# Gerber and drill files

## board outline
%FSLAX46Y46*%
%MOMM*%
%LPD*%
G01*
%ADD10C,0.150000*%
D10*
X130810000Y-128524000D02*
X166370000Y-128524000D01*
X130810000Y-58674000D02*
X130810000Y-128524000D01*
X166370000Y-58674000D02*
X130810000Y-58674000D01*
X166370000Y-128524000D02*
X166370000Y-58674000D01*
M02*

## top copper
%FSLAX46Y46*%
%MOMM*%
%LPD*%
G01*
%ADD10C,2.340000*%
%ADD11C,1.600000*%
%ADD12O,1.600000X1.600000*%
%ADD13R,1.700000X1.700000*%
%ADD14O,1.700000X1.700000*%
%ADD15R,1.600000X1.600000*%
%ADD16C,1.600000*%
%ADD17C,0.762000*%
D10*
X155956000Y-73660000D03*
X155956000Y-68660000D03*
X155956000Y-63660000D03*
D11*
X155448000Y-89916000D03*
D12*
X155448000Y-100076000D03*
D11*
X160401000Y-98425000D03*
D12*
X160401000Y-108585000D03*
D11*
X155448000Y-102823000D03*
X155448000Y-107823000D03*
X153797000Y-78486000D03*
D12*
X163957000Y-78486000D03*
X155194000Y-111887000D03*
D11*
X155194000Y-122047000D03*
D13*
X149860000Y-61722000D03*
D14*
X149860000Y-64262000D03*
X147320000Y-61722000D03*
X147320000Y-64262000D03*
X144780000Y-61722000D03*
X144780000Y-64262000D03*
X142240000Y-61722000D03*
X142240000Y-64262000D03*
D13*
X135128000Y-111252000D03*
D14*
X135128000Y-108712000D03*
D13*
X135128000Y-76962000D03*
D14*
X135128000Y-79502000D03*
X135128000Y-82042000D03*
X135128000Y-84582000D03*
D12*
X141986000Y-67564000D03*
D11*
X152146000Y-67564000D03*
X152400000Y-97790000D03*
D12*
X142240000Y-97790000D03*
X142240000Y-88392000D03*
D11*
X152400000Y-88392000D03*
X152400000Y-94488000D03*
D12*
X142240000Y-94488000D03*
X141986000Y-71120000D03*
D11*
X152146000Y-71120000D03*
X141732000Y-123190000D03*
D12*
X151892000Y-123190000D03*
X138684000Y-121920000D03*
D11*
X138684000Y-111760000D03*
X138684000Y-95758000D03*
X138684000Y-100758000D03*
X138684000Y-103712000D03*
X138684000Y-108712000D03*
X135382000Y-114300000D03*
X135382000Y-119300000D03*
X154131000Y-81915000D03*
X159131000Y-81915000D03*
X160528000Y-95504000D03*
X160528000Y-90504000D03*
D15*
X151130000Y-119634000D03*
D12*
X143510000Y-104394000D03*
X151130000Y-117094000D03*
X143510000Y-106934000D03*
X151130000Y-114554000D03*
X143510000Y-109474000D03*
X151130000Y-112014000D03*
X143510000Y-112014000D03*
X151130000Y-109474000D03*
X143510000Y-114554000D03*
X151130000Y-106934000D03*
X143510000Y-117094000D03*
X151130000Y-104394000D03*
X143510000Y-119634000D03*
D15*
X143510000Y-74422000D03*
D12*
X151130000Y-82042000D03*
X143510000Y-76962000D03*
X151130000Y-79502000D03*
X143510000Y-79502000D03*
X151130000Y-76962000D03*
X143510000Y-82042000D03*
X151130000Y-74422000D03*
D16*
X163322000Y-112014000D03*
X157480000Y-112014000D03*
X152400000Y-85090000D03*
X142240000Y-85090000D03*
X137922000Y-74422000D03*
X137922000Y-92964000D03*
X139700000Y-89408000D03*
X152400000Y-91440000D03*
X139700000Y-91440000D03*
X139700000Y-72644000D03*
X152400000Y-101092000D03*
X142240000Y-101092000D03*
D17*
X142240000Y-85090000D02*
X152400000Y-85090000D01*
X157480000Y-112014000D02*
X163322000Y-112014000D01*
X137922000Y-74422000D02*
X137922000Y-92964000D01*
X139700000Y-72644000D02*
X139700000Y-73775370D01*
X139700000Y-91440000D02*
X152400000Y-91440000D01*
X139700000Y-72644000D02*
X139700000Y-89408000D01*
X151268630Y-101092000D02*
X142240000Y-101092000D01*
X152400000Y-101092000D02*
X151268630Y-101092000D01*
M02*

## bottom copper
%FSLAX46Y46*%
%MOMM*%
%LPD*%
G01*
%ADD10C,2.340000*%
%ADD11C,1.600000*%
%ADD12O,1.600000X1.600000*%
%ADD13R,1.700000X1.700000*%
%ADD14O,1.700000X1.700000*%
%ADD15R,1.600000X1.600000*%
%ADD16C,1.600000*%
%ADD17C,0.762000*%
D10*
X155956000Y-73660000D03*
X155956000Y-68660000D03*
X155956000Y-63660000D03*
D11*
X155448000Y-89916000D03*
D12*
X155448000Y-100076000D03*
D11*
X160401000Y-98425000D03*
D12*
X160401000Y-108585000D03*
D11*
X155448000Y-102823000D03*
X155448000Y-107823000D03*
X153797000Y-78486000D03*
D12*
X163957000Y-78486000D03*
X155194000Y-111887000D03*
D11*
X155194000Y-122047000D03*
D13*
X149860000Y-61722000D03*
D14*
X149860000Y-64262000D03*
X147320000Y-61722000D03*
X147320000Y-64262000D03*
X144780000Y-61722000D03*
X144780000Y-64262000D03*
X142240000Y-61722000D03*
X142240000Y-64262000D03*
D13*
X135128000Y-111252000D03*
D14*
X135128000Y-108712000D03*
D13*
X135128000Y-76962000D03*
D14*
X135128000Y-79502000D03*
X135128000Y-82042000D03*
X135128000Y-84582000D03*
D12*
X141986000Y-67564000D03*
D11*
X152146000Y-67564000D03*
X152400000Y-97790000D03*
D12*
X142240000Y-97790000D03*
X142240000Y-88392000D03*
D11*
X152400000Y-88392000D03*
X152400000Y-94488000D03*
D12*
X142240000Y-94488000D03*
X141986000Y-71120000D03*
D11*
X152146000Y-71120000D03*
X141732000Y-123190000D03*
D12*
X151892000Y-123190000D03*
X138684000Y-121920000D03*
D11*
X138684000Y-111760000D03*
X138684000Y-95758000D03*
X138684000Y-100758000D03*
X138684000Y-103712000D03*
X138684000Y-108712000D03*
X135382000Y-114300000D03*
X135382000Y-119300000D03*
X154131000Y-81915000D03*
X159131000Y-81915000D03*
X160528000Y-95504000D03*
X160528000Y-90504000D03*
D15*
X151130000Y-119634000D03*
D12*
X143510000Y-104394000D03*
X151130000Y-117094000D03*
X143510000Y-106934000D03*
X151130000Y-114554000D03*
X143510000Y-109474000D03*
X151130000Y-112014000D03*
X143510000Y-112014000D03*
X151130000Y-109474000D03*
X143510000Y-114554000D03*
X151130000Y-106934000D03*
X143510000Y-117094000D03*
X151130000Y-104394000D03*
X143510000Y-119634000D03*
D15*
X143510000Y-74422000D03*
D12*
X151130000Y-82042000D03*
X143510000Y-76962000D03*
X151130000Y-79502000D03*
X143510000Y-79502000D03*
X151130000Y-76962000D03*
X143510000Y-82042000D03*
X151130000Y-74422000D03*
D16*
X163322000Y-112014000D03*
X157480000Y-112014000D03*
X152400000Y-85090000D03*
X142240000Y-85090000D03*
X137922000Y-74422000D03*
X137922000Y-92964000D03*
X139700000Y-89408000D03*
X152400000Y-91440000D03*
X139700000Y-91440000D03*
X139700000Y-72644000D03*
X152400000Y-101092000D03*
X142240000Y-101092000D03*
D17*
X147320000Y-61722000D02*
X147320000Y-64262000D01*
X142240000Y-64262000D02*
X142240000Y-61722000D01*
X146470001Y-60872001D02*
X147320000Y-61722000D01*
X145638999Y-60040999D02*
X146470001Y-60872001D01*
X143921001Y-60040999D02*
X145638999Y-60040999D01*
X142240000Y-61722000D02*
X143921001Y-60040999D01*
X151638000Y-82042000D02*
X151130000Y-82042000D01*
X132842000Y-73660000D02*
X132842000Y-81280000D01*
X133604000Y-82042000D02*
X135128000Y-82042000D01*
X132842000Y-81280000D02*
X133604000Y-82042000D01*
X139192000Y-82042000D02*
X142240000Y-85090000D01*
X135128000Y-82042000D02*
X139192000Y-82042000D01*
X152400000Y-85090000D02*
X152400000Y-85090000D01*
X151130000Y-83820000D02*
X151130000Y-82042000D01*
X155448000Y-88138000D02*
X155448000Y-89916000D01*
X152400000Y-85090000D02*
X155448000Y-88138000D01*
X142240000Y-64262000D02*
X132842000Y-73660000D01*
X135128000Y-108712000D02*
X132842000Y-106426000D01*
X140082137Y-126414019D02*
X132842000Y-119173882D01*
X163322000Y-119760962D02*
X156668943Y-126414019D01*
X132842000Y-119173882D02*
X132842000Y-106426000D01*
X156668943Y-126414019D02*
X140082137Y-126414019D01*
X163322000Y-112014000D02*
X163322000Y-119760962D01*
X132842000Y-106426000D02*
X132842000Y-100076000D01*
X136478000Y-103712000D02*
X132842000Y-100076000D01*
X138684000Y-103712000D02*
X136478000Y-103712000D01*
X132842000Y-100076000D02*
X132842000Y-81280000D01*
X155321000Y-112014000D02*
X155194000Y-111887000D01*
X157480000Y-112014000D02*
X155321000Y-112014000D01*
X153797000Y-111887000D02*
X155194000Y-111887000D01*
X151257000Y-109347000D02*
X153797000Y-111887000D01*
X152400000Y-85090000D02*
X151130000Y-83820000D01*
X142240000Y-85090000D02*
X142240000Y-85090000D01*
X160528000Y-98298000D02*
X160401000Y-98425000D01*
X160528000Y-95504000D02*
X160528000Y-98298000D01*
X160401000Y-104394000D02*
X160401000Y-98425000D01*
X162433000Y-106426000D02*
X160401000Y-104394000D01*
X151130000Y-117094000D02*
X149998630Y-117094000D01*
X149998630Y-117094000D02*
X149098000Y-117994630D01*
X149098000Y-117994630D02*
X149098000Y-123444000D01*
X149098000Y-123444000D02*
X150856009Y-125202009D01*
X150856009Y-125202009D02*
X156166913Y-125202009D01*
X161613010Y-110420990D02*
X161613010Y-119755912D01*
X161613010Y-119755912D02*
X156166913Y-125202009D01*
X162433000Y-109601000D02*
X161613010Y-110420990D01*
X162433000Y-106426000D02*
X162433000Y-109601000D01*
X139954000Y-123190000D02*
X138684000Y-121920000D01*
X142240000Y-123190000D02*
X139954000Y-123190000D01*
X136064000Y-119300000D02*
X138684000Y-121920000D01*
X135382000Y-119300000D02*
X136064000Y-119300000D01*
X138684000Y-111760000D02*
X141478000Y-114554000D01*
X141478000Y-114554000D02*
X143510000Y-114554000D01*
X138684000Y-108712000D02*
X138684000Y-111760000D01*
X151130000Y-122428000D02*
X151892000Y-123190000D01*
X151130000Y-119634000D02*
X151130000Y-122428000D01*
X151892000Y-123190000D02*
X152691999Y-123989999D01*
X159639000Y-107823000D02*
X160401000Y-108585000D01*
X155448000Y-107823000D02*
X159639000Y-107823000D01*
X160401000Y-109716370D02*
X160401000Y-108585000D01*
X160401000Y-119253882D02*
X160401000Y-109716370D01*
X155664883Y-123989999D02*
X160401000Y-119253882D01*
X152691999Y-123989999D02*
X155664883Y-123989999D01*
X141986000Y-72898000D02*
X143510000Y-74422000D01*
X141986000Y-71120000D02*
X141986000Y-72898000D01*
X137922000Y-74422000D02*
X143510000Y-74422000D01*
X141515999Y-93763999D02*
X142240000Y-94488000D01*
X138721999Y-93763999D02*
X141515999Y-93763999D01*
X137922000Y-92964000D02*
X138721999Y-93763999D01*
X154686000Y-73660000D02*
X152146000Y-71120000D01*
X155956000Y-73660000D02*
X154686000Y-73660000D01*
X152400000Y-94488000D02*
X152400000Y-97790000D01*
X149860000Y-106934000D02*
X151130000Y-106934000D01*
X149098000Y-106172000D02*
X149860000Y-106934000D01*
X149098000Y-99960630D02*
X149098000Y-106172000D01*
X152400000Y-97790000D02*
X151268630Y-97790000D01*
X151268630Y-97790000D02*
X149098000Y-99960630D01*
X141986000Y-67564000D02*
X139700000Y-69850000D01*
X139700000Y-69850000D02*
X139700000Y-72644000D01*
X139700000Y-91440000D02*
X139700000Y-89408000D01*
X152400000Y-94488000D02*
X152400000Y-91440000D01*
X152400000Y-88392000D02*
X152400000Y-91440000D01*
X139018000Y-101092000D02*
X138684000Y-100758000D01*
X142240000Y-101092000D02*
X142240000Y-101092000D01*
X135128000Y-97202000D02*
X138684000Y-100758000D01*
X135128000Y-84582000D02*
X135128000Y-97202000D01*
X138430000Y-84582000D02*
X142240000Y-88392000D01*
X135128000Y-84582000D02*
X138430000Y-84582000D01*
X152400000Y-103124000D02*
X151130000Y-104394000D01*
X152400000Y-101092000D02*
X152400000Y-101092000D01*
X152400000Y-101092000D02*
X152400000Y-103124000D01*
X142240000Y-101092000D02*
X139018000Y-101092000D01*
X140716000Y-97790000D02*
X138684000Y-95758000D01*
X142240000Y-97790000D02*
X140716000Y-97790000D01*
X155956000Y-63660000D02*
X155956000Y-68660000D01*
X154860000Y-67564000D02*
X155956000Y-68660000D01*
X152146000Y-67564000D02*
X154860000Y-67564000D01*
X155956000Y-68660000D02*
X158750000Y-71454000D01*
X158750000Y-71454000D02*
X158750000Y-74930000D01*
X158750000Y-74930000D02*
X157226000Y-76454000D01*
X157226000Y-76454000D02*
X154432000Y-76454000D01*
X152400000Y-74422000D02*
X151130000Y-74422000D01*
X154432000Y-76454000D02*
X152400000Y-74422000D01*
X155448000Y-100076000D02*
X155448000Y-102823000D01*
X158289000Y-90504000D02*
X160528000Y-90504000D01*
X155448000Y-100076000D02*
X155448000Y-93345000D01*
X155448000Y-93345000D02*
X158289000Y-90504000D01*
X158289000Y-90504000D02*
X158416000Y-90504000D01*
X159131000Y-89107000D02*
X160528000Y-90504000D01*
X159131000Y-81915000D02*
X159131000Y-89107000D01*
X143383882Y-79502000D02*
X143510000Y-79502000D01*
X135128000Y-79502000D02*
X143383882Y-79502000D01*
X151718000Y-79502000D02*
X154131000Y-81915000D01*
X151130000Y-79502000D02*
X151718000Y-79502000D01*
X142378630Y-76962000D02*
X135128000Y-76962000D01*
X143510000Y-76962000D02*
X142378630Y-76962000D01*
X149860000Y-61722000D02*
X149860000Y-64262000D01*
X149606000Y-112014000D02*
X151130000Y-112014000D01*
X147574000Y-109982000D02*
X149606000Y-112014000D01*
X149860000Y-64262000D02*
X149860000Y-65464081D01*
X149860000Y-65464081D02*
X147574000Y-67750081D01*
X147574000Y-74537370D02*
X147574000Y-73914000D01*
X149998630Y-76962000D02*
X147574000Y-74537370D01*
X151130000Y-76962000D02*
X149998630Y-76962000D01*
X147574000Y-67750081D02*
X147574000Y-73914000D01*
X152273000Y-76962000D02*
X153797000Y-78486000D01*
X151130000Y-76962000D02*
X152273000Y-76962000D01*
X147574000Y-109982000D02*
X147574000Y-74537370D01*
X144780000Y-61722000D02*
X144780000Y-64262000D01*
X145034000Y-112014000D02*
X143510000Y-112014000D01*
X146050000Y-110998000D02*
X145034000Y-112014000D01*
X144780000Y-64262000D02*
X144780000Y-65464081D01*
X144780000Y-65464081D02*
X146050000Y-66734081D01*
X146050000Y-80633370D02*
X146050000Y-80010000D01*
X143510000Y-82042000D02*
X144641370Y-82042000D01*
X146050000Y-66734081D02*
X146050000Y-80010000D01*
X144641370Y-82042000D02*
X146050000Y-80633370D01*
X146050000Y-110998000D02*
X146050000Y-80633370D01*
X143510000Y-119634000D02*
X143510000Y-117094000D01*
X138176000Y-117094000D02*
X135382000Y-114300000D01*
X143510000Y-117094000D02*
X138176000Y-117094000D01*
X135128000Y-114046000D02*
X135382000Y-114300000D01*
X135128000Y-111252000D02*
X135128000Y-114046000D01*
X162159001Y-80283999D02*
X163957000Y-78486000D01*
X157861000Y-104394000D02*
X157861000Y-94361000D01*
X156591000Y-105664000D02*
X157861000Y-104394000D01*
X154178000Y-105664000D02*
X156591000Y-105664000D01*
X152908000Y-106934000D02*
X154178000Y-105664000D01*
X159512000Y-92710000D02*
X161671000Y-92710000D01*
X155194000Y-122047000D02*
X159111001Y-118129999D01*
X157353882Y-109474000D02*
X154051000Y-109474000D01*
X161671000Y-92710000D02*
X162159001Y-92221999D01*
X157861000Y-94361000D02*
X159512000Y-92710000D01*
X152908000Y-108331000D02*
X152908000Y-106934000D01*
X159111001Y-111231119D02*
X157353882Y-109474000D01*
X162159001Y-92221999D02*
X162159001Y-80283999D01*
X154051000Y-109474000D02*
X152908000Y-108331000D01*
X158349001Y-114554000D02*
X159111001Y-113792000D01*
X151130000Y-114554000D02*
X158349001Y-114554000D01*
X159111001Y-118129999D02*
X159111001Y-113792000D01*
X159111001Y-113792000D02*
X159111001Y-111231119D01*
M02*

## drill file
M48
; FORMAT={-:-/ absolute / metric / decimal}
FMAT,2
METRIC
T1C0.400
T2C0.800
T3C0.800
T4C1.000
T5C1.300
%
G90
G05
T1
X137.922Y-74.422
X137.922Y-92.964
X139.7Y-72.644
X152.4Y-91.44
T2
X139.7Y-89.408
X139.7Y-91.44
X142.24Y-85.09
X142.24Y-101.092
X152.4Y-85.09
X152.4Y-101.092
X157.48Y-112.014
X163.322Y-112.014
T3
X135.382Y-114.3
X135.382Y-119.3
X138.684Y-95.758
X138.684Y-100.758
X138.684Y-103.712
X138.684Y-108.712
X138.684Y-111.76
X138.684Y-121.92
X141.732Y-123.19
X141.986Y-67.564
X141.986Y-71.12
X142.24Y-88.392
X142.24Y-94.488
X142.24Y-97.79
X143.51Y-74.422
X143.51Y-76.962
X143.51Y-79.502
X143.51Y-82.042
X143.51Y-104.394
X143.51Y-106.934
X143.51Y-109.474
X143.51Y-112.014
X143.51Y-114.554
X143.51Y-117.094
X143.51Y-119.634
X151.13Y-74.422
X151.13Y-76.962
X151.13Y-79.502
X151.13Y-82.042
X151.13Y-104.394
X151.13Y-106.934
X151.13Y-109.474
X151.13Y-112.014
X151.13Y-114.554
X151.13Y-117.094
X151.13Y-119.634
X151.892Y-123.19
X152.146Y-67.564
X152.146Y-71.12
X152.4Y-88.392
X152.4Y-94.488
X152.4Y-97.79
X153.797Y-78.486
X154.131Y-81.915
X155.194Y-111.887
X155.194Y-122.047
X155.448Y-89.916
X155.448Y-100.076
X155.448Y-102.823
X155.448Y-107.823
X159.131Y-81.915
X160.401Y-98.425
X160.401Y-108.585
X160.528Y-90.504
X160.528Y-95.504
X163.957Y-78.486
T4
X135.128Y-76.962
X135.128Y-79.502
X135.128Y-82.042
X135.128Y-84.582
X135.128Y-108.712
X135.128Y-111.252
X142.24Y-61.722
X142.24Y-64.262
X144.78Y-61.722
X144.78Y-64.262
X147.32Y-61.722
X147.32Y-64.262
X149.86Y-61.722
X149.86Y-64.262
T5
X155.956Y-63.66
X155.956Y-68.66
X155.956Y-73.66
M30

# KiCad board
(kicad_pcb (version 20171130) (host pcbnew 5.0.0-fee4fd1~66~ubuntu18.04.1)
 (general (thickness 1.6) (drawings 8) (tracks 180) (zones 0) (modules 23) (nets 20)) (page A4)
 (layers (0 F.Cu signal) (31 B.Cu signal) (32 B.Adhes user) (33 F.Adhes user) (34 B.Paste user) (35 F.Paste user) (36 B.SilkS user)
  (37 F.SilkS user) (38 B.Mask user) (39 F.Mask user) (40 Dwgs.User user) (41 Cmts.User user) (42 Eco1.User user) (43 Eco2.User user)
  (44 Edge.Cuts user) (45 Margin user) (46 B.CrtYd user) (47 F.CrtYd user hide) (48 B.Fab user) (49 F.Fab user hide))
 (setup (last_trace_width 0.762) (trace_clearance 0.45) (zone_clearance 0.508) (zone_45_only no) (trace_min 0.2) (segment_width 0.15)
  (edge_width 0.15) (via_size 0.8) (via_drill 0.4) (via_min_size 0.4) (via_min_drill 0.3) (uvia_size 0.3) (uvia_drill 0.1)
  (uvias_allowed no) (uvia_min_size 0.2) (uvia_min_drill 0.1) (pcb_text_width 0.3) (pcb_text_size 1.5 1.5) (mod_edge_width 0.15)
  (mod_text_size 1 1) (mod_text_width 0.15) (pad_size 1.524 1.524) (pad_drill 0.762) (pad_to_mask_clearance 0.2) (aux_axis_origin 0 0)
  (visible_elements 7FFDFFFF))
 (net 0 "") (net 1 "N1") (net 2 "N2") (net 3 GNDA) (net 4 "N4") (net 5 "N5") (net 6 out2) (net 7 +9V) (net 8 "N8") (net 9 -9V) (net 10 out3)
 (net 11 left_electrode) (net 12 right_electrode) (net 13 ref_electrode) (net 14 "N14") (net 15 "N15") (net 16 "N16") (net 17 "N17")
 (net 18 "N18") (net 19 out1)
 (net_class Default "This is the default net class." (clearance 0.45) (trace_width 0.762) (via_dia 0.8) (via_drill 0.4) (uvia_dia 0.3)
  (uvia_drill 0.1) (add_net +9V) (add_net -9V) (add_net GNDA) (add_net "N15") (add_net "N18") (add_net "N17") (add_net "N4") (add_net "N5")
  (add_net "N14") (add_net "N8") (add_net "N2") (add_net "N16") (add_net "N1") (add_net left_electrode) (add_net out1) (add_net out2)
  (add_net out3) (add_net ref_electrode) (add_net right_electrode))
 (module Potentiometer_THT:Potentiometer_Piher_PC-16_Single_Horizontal (layer F.Cu) (at 155.956 73.66)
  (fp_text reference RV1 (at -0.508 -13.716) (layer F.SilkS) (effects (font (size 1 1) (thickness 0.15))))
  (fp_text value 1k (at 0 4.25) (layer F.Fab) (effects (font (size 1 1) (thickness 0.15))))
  (pad 1 thru_hole circle (at 0 0) (size 2.34 2.34) (drill 1.3) (layers *.Cu *.Mask) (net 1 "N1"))
  (pad 2 thru_hole circle (at 0 -5) (size 2.34 2.34) (drill 1.3) (layers *.Cu *.Mask) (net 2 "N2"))
  (pad 3 thru_hole circle (at 0 -10) (size 2.34 2.34) (drill 1.3) (layers *.Cu *.Mask) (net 2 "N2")))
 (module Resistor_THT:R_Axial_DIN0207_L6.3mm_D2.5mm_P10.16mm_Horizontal (layer F.Cu) (at 155.448 89.916 270)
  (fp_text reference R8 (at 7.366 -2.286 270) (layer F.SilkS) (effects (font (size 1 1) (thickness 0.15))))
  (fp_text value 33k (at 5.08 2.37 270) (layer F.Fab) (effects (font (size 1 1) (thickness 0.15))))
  (pad 1 thru_hole circle (at 0 0 270) (size 1.6 1.6) (drill 0.8) (layers *.Cu *.Mask) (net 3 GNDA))
  (pad 2 thru_hole oval (at 10.16 0 270) (size 1.6 1.6) (drill 0.8) (layers *.Cu *.Mask) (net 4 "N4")))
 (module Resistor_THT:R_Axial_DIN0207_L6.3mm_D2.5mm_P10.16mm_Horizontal (layer F.Cu) (at 160.401 98.425 270)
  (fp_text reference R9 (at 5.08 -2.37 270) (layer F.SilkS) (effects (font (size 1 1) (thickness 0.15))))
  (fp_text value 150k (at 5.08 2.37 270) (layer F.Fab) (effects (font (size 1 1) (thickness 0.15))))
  (pad 1 thru_hole circle (at 0 0 270) (size 1.6 1.6) (drill 0.8) (layers *.Cu *.Mask) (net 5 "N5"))
  (pad 2 thru_hole oval (at 10.16 0 270) (size 1.6 1.6) (drill 0.8) (layers *.Cu *.Mask) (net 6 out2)))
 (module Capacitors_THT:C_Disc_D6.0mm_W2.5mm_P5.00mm (layer F.Cu) (at 155.448 107.823 90)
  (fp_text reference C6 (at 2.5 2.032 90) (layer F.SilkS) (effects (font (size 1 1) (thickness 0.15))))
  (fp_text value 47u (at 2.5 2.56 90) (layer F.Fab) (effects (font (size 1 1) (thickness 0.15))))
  (pad 2 thru_hole circle (at 5 0 90) (size 1.6 1.6) (drill 0.8) (layers *.Cu *.Mask) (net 4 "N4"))
  (pad 1 thru_hole circle (at 0 0 90) (size 1.6 1.6) (drill 0.8) (layers *.Cu *.Mask) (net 6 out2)))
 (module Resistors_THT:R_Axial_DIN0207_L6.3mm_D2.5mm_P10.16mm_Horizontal (layer F.Cu) (at 153.797 78.486)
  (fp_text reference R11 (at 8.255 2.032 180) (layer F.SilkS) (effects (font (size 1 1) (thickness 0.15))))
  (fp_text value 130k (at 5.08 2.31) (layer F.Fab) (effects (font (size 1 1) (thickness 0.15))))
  (pad 1 thru_hole circle (at 0 0) (size 1.6 1.6) (drill 0.8) (layers *.Cu *.Mask) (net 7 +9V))
  (pad 2 thru_hole oval (at 10.16 0) (size 1.6 1.6) (drill 0.8) (layers *.Cu *.Mask) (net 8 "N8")))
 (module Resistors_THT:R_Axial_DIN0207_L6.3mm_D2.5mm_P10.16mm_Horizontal (layer F.Cu) (at 155.194 122.047 90)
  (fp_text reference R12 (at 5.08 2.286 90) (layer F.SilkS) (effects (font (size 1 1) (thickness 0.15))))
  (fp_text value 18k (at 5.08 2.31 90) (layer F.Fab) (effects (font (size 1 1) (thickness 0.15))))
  (pad 2 thru_hole oval (at 10.16 0 90) (size 1.6 1.6) (drill 0.8) (layers *.Cu *.Mask) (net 3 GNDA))
  (pad 1 thru_hole circle (at 0 0 90) (size 1.6 1.6) (drill 0.8) (layers *.Cu *.Mask) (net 8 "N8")))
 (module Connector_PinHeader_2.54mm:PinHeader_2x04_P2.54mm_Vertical (layer F.Cu) (at 149.86 61.722 270)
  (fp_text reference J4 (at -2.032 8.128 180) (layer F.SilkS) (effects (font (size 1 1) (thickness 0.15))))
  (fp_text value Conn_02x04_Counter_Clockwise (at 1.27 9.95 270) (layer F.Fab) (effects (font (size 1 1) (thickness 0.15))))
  (pad 1 thru_hole rect (at 0 0 270) (size 1.7 1.7) (drill 1) (layers *.Cu *.Mask) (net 7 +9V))
  (pad 2 thru_hole oval (at 2.54 0 270) (size 1.7 1.7) (drill 1) (layers *.Cu *.Mask) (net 7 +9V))
  (pad 3 thru_hole oval (at 0 2.54 270) (size 1.7 1.7) (drill 1) (layers *.Cu *.Mask) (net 3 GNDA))
  (pad 4 thru_hole oval (at 2.54 2.54 270) (size 1.7 1.7) (drill 1) (layers *.Cu *.Mask) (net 3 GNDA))
  (pad 5 thru_hole oval (at 0 5.08 270) (size 1.7 1.7) (drill 1) (layers *.Cu *.Mask) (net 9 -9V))
  (pad 6 thru_hole oval (at 2.54 5.08 270) (size 1.7 1.7) (drill 1) (layers *.Cu *.Mask) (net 9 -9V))
  (pad 7 thru_hole oval (at 0 7.62 270) (size 1.7 1.7) (drill 1) (layers *.Cu *.Mask) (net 3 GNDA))
  (pad 8 thru_hole oval (at 2.54 7.62 270) (size 1.7 1.7) (drill 1) (layers *.Cu *.Mask) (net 3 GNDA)))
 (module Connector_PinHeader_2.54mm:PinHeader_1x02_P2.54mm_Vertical (layer F.Cu) (at 135.128 111.252 180)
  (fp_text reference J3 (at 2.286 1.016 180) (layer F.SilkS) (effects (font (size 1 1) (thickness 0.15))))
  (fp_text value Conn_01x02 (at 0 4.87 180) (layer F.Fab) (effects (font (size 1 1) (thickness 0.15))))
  (pad 1 thru_hole rect (at 0 0 180) (size 1.7 1.7) (drill 1) (layers *.Cu *.Mask) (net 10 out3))
  (pad 2 thru_hole oval (at 0 2.54 180) (size 1.7 1.7) (drill 1) (layers *.Cu *.Mask) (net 3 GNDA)))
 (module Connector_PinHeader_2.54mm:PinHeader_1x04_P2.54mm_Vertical (layer F.Cu) (at 135.128 76.962)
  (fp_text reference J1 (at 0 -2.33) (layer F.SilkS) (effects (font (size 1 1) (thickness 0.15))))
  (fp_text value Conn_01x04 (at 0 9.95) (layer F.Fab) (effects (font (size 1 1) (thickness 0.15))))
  (pad 1 thru_hole rect (at 0 0) (size 1.7 1.7) (drill 1) (layers *.Cu *.Mask) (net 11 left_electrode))
  (pad 2 thru_hole oval (at 0 2.54) (size 1.7 1.7) (drill 1) (layers *.Cu *.Mask) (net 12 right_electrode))
  (pad 3 thru_hole oval (at 0 5.08) (size 1.7 1.7) (drill 1) (layers *.Cu *.Mask) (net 3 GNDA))
  (pad 4 thru_hole oval (at 0 7.62) (size 1.7 1.7) (drill 1) (layers *.Cu *.Mask) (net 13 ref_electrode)))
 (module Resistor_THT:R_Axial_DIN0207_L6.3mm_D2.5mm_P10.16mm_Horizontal (layer F.Cu) (at 152.146 67.564 180)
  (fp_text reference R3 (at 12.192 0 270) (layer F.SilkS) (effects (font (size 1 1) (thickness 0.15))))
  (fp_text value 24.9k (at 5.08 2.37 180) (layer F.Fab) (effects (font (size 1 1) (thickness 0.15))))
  (pad 2 thru_hole oval (at 10.16 0 180) (size 1.6 1.6) (drill 0.8) (layers *.Cu *.Mask) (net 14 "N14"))
  (pad 1 thru_hole circle (at 0 0 180) (size 1.6 1.6) (drill 0.8) (layers *.Cu *.Mask) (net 2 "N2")))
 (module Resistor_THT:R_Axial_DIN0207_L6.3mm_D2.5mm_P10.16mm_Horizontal (layer F.Cu) (at 152.4 97.79 180)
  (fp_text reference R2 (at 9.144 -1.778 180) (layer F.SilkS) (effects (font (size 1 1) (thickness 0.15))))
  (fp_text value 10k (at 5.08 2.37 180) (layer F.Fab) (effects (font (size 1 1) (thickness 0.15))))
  (pad 1 thru_hole circle (at 0 0 180) (size 1.6 1.6) (drill 0.8) (layers *.Cu *.Mask) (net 14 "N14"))
  (pad 2 thru_hole oval (at 10.16 0 180) (size 1.6 1.6) (drill 0.8) (layers *.Cu *.Mask) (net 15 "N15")))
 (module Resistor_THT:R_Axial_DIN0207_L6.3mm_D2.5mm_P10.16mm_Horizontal (layer F.Cu) (at 152.4 88.392 180)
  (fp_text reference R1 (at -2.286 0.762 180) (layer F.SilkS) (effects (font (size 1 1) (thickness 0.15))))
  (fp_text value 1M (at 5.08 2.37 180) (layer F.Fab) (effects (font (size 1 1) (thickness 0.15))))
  (pad 2 thru_hole oval (at 10.16 0 180) (size 1.6 1.6) (drill 0.8) (layers *.Cu *.Mask) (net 13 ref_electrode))
  (pad 1 thru_hole circle (at 0 0 180) (size 1.6 1.6) (drill 0.8) (layers *.Cu *.Mask) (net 14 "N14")))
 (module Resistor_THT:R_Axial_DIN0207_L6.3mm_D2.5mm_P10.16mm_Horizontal (layer F.Cu) (at 152.4 94.488 180)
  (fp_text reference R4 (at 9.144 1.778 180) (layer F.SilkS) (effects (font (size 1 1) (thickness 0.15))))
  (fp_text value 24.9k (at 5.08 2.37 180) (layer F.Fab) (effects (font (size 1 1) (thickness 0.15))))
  (pad 1 thru_hole circle (at 0 0 180) (size 1.6 1.6) (drill 0.8) (layers *.Cu *.Mask) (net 14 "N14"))
  (pad 2 thru_hole oval (at 10.16 0 180) (size 1.6 1.6) (drill 0.8) (layers *.Cu *.Mask) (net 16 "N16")))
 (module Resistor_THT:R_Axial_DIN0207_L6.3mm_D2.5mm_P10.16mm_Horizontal (layer F.Cu) (at 152.146 71.12 180)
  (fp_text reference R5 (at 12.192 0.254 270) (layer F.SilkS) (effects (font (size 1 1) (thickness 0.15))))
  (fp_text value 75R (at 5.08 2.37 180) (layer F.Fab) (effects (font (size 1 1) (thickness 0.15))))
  (pad 2 thru_hole oval (at 10.16 0 180) (size 1.6 1.6) (drill 0.8) (layers *.Cu *.Mask) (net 16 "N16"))
  (pad 1 thru_hole circle (at 0 0 180) (size 1.6 1.6) (drill 0.8) (layers *.Cu *.Mask) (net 1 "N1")))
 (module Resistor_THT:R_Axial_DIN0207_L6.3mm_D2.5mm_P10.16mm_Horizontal (layer F.Cu) (at 141.732 123.19)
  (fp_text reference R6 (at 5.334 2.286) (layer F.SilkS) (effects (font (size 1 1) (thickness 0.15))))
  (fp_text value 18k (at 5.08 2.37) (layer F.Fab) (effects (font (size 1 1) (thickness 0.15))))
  (pad 1 thru_hole circle (at 0 0) (size 1.6 1.6) (drill 0.8) (layers *.Cu *.Mask) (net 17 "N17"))
  (pad 2 thru_hole oval (at 10.16 0) (size 1.6 1.6) (drill 0.8) (layers *.Cu *.Mask) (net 6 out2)))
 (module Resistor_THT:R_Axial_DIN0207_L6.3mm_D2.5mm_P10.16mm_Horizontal (layer F.Cu) (at 138.684 111.76 270)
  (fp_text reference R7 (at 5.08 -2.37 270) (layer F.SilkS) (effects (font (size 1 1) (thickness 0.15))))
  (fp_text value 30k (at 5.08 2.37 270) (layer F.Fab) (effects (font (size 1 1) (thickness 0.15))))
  (pad 2 thru_hole oval (at 10.16 0 270) (size 1.6 1.6) (drill 0.8) (layers *.Cu *.Mask) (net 17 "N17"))
  (pad 1 thru_hole circle (at 0 0 270) (size 1.6 1.6) (drill 0.8) (layers *.Cu *.Mask) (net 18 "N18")))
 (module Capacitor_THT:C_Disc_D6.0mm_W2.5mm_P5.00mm (layer F.Cu) (at 138.684 95.758 270)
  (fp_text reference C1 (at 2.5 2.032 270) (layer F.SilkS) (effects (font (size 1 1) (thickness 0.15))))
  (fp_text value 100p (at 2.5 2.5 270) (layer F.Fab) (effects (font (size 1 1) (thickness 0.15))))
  (pad 1 thru_hole circle (at 0 0 270) (size 1.6 1.6) (drill 0.8) (layers *.Cu *.Mask) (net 15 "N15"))
  (pad 2 thru_hole circle (at 5 0 270) (size 1.6 1.6) (drill 0.8) (layers *.Cu *.Mask) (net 13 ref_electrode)))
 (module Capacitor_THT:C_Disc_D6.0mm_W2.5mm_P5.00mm (layer F.Cu) (at 138.684 108.712 90)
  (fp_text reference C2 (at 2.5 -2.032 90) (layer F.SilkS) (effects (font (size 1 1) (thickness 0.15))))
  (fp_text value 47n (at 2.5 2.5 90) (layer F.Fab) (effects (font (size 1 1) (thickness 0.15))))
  (pad 2 thru_hole circle (at 5 0 90) (size 1.6 1.6) (drill 0.8) (layers *.Cu *.Mask) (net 3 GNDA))
  (pad 1 thru_hole circle (at 0 0 90) (size 1.6 1.6) (drill 0.8) (layers *.Cu *.Mask) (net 18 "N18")))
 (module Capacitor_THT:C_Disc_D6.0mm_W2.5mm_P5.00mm (layer F.Cu) (at 135.382 114.3 270)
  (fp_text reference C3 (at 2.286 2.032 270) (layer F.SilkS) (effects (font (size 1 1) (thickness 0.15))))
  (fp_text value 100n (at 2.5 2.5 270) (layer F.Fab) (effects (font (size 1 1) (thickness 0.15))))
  (pad 1 thru_hole circle (at 0 0 270) (size 1.6 1.6) (drill 0.8) (layers *.Cu *.Mask) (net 10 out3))
  (pad 2 thru_hole circle (at 5 0 270) (size 1.6 1.6) (drill 0.8) (layers *.Cu *.Mask) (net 17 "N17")))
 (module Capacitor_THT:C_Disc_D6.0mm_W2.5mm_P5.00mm (layer F.Cu) (at 159.131 81.915 180)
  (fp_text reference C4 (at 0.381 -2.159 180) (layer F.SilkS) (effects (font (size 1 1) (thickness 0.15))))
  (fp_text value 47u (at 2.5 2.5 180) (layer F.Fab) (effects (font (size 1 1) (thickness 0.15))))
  (pad 2 thru_hole circle (at 5 0 180) (size 1.6 1.6) (drill 0.8) (layers *.Cu *.Mask) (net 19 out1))
  (pad 1 thru_hole circle (at 0 0 180) (size 1.6 1.6) (drill 0.8) (layers *.Cu *.Mask) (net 4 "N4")))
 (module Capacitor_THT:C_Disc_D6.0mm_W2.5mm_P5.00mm (layer F.Cu) (at 160.528 95.504 90)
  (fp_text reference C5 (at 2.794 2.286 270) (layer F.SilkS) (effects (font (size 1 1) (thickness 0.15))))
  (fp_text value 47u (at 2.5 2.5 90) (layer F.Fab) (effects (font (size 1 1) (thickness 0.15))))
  (pad 1 thru_hole circle (at 0 0 90) (size 1.6 1.6) (drill 0.8) (layers *.Cu *.Mask) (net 5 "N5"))
  (pad 2 thru_hole circle (at 5 0 90) (size 1.6 1.6) (drill 0.8) (layers *.Cu *.Mask) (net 4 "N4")))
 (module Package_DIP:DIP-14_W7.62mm (layer F.Cu) (at 151.13 119.634 180)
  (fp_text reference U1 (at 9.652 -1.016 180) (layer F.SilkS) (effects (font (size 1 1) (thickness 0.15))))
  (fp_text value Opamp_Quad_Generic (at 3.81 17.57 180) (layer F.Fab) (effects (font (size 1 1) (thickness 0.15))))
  (pad 1 thru_hole rect (at 0 0 180) (size 1.6 1.6) (drill 0.8) (layers *.Cu *.Mask) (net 6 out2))
  (pad 8 thru_hole oval (at 7.62 15.24 180) (size 1.6 1.6) (drill 0.8) (layers *.Cu *.Mask))
  (pad 2 thru_hole oval (at 0 2.54 180) (size 1.6 1.6) (drill 0.8) (layers *.Cu *.Mask) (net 5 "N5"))
  (pad 9 thru_hole oval (at 7.62 12.7 180) (size 1.6 1.6) (drill 0.8) (layers *.Cu *.Mask))
  (pad 3 thru_hole oval (at 0 5.08 180) (size 1.6 1.6) (drill 0.8) (layers *.Cu *.Mask) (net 8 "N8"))
  (pad 10 thru_hole oval (at 7.62 10.16 180) (size 1.6 1.6) (drill 0.8) (layers *.Cu *.Mask))
  (pad 4 thru_hole oval (at 0 7.62 180) (size 1.6 1.6) (drill 0.8) (layers *.Cu *.Mask) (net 7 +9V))
  (pad 11 thru_hole oval (at 7.62 7.62 180) (size 1.6 1.6) (drill 0.8) (layers *.Cu *.Mask) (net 9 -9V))
  (pad 5 thru_hole oval (at 0 10.16 180) (size 1.6 1.6) (drill 0.8) (layers *.Cu *.Mask) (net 3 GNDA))
  (pad 12 thru_hole oval (at 7.62 5.08 180) (size 1.6 1.6) (drill 0.8) (layers *.Cu *.Mask) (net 18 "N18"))
  (pad 6 thru_hole oval (at 0 12.7 180) (size 1.6 1.6) (drill 0.8) (layers *.Cu *.Mask) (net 14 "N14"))
  (pad 13 thru_hole oval (at 7.62 2.54 180) (size 1.6 1.6) (drill 0.8) (layers *.Cu *.Mask) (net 10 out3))
  (pad 7 thru_hole oval (at 0 15.24 180) (size 1.6 1.6) (drill 0.8) (layers *.Cu *.Mask) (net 13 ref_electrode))
  (pad 14 thru_hole oval (at 7.62 0 180) (size 1.6 1.6) (drill 0.8) (layers *.Cu *.Mask) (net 10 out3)))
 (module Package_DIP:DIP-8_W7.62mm (layer F.Cu) (at 143.51 74.422)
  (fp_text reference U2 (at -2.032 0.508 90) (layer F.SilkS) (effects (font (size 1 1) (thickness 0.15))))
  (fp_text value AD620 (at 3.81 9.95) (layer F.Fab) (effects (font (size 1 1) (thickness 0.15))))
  (pad 1 thru_hole rect (at 0 0) (size 1.6 1.6) (drill 0.8) (layers *.Cu *.Mask) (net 16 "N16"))
  (pad 5 thru_hole oval (at 7.62 7.62) (size 1.6 1.6) (drill 0.8) (layers *.Cu *.Mask) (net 3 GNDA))
  (pad 2 thru_hole oval (at 0 2.54) (size 1.6 1.6) (drill 0.8) (layers *.Cu *.Mask) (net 11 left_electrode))
  (pad 6 thru_hole oval (at 7.62 5.08) (size 1.6 1.6) (drill 0.8) (layers *.Cu *.Mask) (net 19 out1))
  (pad 3 thru_hole oval (at 0 5.08) (size 1.6 1.6) (drill 0.8) (layers *.Cu *.Mask) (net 12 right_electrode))
  (pad 7 thru_hole oval (at 7.62 2.54) (size 1.6 1.6) (drill 0.8) (layers *.Cu *.Mask) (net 7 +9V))
  (pad 4 thru_hole oval (at 0 7.62) (size 1.6 1.6) (drill 0.8) (layers *.Cu *.Mask) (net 9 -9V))
  (pad 8 thru_hole oval (at 7.62 0) (size 1.6 1.6) (drill 0.8) (layers *.Cu *.Mask) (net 2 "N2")))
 (gr_line (start 130.81 128.524) (end 166.37 128.524) (layer Edge.Cuts) (width 0.15))
 (gr_line (start 130.81 58.674) (end 130.81 128.524) (layer Edge.Cuts) (width 0.15))
 (gr_line (start 166.37 58.674) (end 130.81 58.674) (layer Edge.Cuts) (width 0.15))
 (gr_line (start 166.37 128.524) (end 166.37 58.674) (layer Edge.Cuts) (width 0.15))
 (via (at 163.322 112.014) (size 1.6) (drill 0.8) (layers F.Cu B.Cu) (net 3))
 (via (at 157.48 112.014) (size 1.6) (drill 0.8) (layers F.Cu B.Cu) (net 3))
 (segment (start 147.32 61.722) (end 147.32 64.262) (width 0.762) (layer B.Cu) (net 3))
 (segment (start 142.24 64.262) (end 142.24 61.722) (width 0.762) (layer B.Cu) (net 3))
 (segment (start 146.470001 60.872001) (end 147.32 61.722) (width 0.762) (layer B.Cu) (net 3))
 (segment (start 145.638999 60.040999) (end 146.470001 60.872001) (width 0.762) (layer B.Cu) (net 3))
 (segment (start 143.921001 60.040999) (end 145.638999 60.040999) (width 0.762) (layer B.Cu) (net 3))
 (segment (start 142.24 61.722) (end 143.921001 60.040999) (width 0.762) (layer B.Cu) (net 3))
 (segment (start 151.638 82.042) (end 151.13 82.042) (width 0.762) (layer B.Cu) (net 3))
 (segment (start 132.842 73.66) (end 132.842 81.28) (width 0.762) (layer B.Cu) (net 3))
 (segment (start 133.604 82.042) (end 135.128 82.042) (width 0.762) (layer B.Cu) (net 3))
 (segment (start 132.842 81.28) (end 133.604 82.042) (width 0.762) (layer B.Cu) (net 3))
 (segment (start 139.192 82.042) (end 142.24 85.09) (width 0.762) (layer B.Cu) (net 3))
 (segment (start 135.128 82.042) (end 139.192 82.042) (width 0.762) (layer B.Cu) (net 3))
 (segment (start 152.4 85.09) (end 152.4 85.09) (width 0.762) (layer B.Cu) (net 3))
 (segment (start 151.13 83.82) (end 151.13 82.042) (width 0.762) (layer B.Cu) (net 3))
 (segment (start 155.448 88.138) (end 155.448 89.916) (width 0.762) (layer B.Cu) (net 3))
 (segment (start 152.4 85.09) (end 155.448 88.138) (width 0.762) (layer B.Cu) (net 3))
 (segment (start 142.24 85.09) (end 152.4 85.09) (width 0.762) (layer F.Cu) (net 3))
 (segment (start 142.24 64.262) (end 132.842 73.66) (width 0.762) (layer B.Cu) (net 3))
 (segment (start 135.128 108.712) (end 132.842 106.426) (width 0.762) (layer B.Cu) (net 3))
 (segment (start 140.082137 126.414019) (end 132.842 119.173882) (width 0.762) (layer B.Cu) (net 3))
 (segment (start 163.322 119.760962) (end 156.668943 126.414019) (width 0.762) (layer B.Cu) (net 3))
 (segment (start 132.842 119.173882) (end 132.842 106.426) (width 0.762) (layer B.Cu) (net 3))
 (segment (start 156.668943 126.414019) (end 140.082137 126.414019) (width 0.762) (layer B.Cu) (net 3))
 (segment (start 163.322 112.014) (end 163.322 119.760962) (width 0.762) (layer B.Cu) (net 3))
 (segment (start 132.842 106.426) (end 132.842 100.076) (width 0.762) (layer B.Cu) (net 3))
 (segment (start 136.478 103.712) (end 132.842 100.076) (width 0.762) (layer B.Cu) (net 3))
 (segment (start 138.684 103.712) (end 136.478 103.712) (width 0.762) (layer B.Cu) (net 3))
 (segment (start 132.842 100.076) (end 132.842 81.28) (width 0.762) (layer B.Cu) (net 3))
 (segment (start 155.321 112.014) (end 155.194 111.887) (width 0.762) (layer B.Cu) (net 3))
 (segment (start 157.48 112.014) (end 155.321 112.014) (width 0.762) (layer B.Cu) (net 3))
 (segment (start 153.797 111.887) (end 155.194 111.887) (width 0.762) (layer B.Cu) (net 3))
 (segment (start 151.257 109.347) (end 153.797 111.887) (width 0.762) (layer B.Cu) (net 3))
 (segment (start 157.48 112.014) (end 163.322 112.014) (width 0.762) (layer F.Cu) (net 3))
 (segment (start 152.4 85.09) (end 151.13 83.82) (width 0.762) (layer B.Cu) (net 3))
 (via (at 152.4 85.09) (size 1.6) (drill 0.8) (layers F.Cu B.Cu) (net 3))
 (segment (start 142.24 85.09) (end 142.24 85.09) (width 0.762) (layer B.Cu) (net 3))
 (via (at 142.24 85.09) (size 1.6) (drill 0.8) (layers F.Cu B.Cu) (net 3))
 (segment (start 160.528 98.298) (end 160.401 98.425) (width 0.762) (layer B.Cu) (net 5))
 (segment (start 160.528 95.504) (end 160.528 98.298) (width 0.762) (layer B.Cu) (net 5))
 (segment (start 160.401 104.394) (end 160.401 98.425) (width 0.762) (layer B.Cu) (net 5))
 (segment (start 162.433 106.426) (end 160.401 104.394) (width 0.762) (layer B.Cu) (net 5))
 (segment (start 151.13 117.094) (end 149.99863 117.094) (width 0.762) (layer B.Cu) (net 5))
 (segment (start 149.99863 117.094) (end 149.098 117.99463) (width 0.762) (layer B.Cu) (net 5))
 (segment (start 149.098 117.99463) (end 149.098 123.444) (width 0.762) (layer B.Cu) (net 5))
 (segment (start 149.098 123.444) (end 150.856009 125.202009) (width 0.762) (layer B.Cu) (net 5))
 (segment (start 150.856009 125.202009) (end 156.166913 125.202009) (width 0.762) (layer B.Cu) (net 5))
 (segment (start 161.61301 110.42099) (end 161.61301 119.755912) (width 0.762) (layer B.Cu) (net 5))
 (segment (start 161.61301 119.755912) (end 156.166913 125.202009) (width 0.762) (layer B.Cu) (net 5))
 (segment (start 162.433 109.601) (end 161.61301 110.42099) (width 0.762) (layer B.Cu) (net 5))
 (segment (start 162.433 106.426) (end 162.433 109.601) (width 0.762) (layer B.Cu) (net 5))
 (segment (start 139.954 123.19) (end 138.684 121.92) (width 0.762) (layer B.Cu) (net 17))
 (segment (start 142.24 123.19) (end 139.954 123.19) (width 0.762) (layer B.Cu) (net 17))
 (segment (start 136.064 119.3) (end 138.684 121.92) (width 0.762) (layer B.Cu) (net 17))
 (segment (start 135.382 119.3) (end 136.064 119.3) (width 0.762) (layer B.Cu) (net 17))
 (segment (start 138.684 111.76) (end 141.478 114.554) (width 0.762) (layer B.Cu) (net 18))
 (segment (start 141.478 114.554) (end 143.51 114.554) (width 0.762) (layer B.Cu) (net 18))
 (segment (start 138.684 108.712) (end 138.684 111.76) (width 0.762) (layer B.Cu) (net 18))
 (segment (start 151.13 122.428) (end 151.892 123.19) (width 0.762) (layer B.Cu) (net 6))
 (segment (start 151.13 119.634) (end 151.13 122.428) (width 0.762) (layer B.Cu) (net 6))
 (segment (start 151.892 123.19) (end 152.691999 123.989999) (width 0.762) (layer B.Cu) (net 6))
 (segment (start 159.639 107.823) (end 160.401 108.585) (width 0.762) (layer B.Cu) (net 6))
 (segment (start 155.448 107.823) (end 159.639 107.823) (width 0.762) (layer B.Cu) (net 6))
 (segment (start 160.401 109.71637) (end 160.401 108.585) (width 0.762) (layer B.Cu) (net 6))
 (segment (start 160.401 119.253882) (end 160.401 109.71637) (width 0.762) (layer B.Cu) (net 6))
 (segment (start 155.664883 123.989999) (end 160.401 119.253882) (width 0.762) (layer B.Cu) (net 6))
 (segment (start 152.691999 123.989999) (end 155.664883 123.989999) (width 0.762) (layer B.Cu) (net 6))
 (segment (start 141.986 72.898) (end 143.51 74.422) (width 0.762) (layer B.Cu) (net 16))
 (segment (start 141.986 71.12) (end 141.986 72.898) (width 0.762) (layer B.Cu) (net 16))
 (segment (start 137.922 74.422) (end 137.922 92.964) (width 0.762) (layer F.Cu) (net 16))
 (via (at 137.922 74.422) (size 1.6) (drill 0.4) (layers F.Cu B.Cu) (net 16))
 (via (at 137.922 92.964) (size 1.6) (drill 0.4) (layers F.Cu B.Cu) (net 16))
 (segment (start 137.922 74.422) (end 143.51 74.422) (width 0.762) (layer B.Cu) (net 16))
 (segment (start 141.515999 93.763999) (end 142.24 94.488) (width 0.762) (layer B.Cu) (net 16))
 (segment (start 138.721999 93.763999) (end 141.515999 93.763999) (width 0.762) (layer B.Cu) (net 16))
 (segment (start 137.922 92.964) (end 138.721999 93.763999) (width 0.762) (layer B.Cu) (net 16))
 (segment (start 154.686 73.66) (end 152.146 71.12) (width 0.762) (layer B.Cu) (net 1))
 (segment (start 155.956 73.66) (end 154.686 73.66) (width 0.762) (layer B.Cu) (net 1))
 (via (at 139.7 89.408) (size 1.6) (drill 0.8) (layers F.Cu B.Cu) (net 14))
 (via (at 152.4 91.44) (size 1.6) (drill 0.4) (layers F.Cu B.Cu) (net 14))
 (segment (start 152.4 94.488) (end 152.4 97.79) (width 0.762) (layer B.Cu) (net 14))
 (segment (start 149.86 106.934) (end 151.13 106.934) (width 0.762) (layer B.Cu) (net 14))
 (segment (start 149.098 106.172) (end 149.86 106.934) (width 0.762) (layer B.Cu) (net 14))
 (segment (start 149.098 99.96063) (end 149.098 106.172) (width 0.762) (layer B.Cu) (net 14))
 (segment (start 152.4 97.79) (end 151.26863 97.79) (width 0.762) (layer B.Cu) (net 14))
 (segment (start 151.26863 97.79) (end 149.098 99.96063) (width 0.762) (layer B.Cu) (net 14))
 (via (at 139.7 91.44) (size 1.6) (drill 0.8) (layers F.Cu B.Cu) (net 14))
 (via (at 139.7 72.644) (size 1.6) (drill 0.4) (layers F.Cu B.Cu) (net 14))
 (segment (start 141.986 67.564) (end 139.7 69.85) (width 0.762) (layer B.Cu) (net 14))
 (segment (start 139.7 72.644) (end 139.7 73.77537) (width 0.762) (layer F.Cu) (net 14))
 (segment (start 139.7 69.85) (end 139.7 72.644) (width 0.762) (layer B.Cu) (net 14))
 (segment (start 139.7 91.44) (end 139.7 89.408) (width 0.762) (layer B.Cu) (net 14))
 (segment (start 139.7 91.44) (end 152.4 91.44) (width 0.762) (layer F.Cu) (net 14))
 (segment (start 139.7 72.644) (end 139.7 89.408) (width 0.762) (layer F.Cu) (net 14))
 (segment (start 152.4 94.488) (end 152.4 91.44) (width 0.762) (layer B.Cu) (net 14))
 (segment (start 152.4 88.392) (end 152.4 91.44) (width 0.762) (layer B.Cu) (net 14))
 (segment (start 139.018 101.092) (end 138.684 100.758) (width 0.762) (layer B.Cu) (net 13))
 (segment (start 142.24 101.092) (end 142.24 101.092) (width 0.762) (layer B.Cu) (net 13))
 (segment (start 135.128 97.202) (end 138.684 100.758) (width 0.762) (layer B.Cu) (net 13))
 (segment (start 135.128 84.582) (end 135.128 97.202) (width 0.762) (layer B.Cu) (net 13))
 (segment (start 138.43 84.582) (end 142.24 88.392) (width 0.762) (layer B.Cu) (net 13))
 (segment (start 135.128 84.582) (end 138.43 84.582) (width 0.762) (layer B.Cu) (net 13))
 (segment (start 152.4 103.124) (end 151.13 104.394) (width 0.762) (layer B.Cu) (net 13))
 (segment (start 152.4 101.092) (end 152.4 101.092) (width 0.762) (layer B.Cu) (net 13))
 (segment (start 152.4 101.092) (end 152.4 103.124) (width 0.762) (layer B.Cu) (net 13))
 (via (at 152.4 101.092) (size 1.6) (drill 0.8) (layers F.Cu B.Cu) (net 13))
 (segment (start 142.24 101.092) (end 139.018 101.092) (width 0.762) (layer B.Cu) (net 13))
 (via (at 142.24 101.092) (size 1.6) (drill 0.8) (layers F.Cu B.Cu) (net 13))
 (segment (start 151.26863 101.092) (end 142.24 101.092) (width 0.762) (layer F.Cu) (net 13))
 (segment (start 152.4 101.092) (end 151.26863 101.092) (width 0.762) (layer F.Cu) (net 13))
 (segment (start 140.716 97.79) (end 138.684 95.758) (width 0.762) (layer B.Cu) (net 15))
 (segment (start 142.24 97.79) (end 140.716 97.79) (width 0.762) (layer B.Cu) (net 15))
 (segment (start 155.956 63.66) (end 155.956 68.66) (width 0.762) (layer B.Cu) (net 2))
 (segment (start 154.86 67.564) (end 155.956 68.66) (width 0.762) (layer B.Cu) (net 2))
 (segment (start 152.146 67.564) (end 154.86 67.564) (width 0.762) (layer B.Cu) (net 2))
 (segment (start 155.956 68.66) (end 158.75 71.454) (width 0.762) (layer B.Cu) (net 2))
 (segment (start 158.75 71.454) (end 158.75 74.93) (width 0.762) (layer B.Cu) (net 2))
 (segment (start 158.75 74.93) (end 157.226 76.454) (width 0.762) (layer B.Cu) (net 2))
 (segment (start 157.226 76.454) (end 154.432 76.454) (width 0.762) (layer B.Cu) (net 2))
 (segment (start 152.4 74.422) (end 151.13 74.422) (width 0.762) (layer B.Cu) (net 2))
 (segment (start 154.432 76.454) (end 152.4 74.422) (width 0.762) (layer B.Cu) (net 2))
 (segment (start 155.448 100.076) (end 155.448 102.823) (width 0.762) (layer B.Cu) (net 4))
 (segment (start 158.289 90.504) (end 160.528 90.504) (width 0.762) (layer B.Cu) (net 4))
 (segment (start 155.448 100.076) (end 155.448 93.345) (width 0.762) (layer B.Cu) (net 4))
 (segment (start 155.448 93.345) (end 158.289 90.504) (width 0.762) (layer B.Cu) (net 4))
 (segment (start 158.289 90.504) (end 158.416 90.504) (width 0.762) (layer B.Cu) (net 4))
 (segment (start 159.131 89.107) (end 160.528 90.504) (width 0.762) (layer B.Cu) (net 4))
 (segment (start 159.131 81.915) (end 159.131 89.107) (width 0.762) (layer B.Cu) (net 4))
 (segment (start 143.383882 79.502) (end 143.51 79.502) (width 0.762) (layer B.Cu) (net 12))
 (segment (start 135.128 79.502) (end 143.383882 79.502) (width 0.762) (layer B.Cu) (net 12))
 (segment (start 151.718 79.502) (end 154.131 81.915) (width 0.762) (layer B.Cu) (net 19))
 (segment (start 151.13 79.502) (end 151.718 79.502) (width 0.762) (layer B.Cu) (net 19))
 (segment (start 142.37863 76.962) (end 135.128 76.962) (width 0.762) (layer B.Cu) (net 11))
 (segment (start 143.51 76.962) (end 142.37863 76.962) (width 0.762) (layer B.Cu) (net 11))
 (segment (start 149.86 61.722) (end 149.86 64.262) (width 0.762) (layer B.Cu) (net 7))
 (segment (start 149.606 112.014) (end 151.13 112.014) (width 0.762) (layer B.Cu) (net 7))
 (segment (start 147.574 109.982) (end 149.606 112.014) (width 0.762) (layer B.Cu) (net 7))
 (segment (start 149.86 64.262) (end 149.86 65.464081) (width 0.762) (layer B.Cu) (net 7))
 (segment (start 149.86 65.464081) (end 147.574 67.750081) (width 0.762) (layer B.Cu) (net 7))
 (segment (start 147.574 74.53737) (end 147.574 73.914) (width 0.762) (layer B.Cu) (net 7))
 (segment (start 149.99863 76.962) (end 147.574 74.53737) (width 0.762) (layer B.Cu) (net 7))
 (segment (start 151.13 76.962) (end 149.99863 76.962) (width 0.762) (layer B.Cu) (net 7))
 (segment (start 147.574 67.750081) (end 147.574 73.914) (width 0.762) (layer B.Cu) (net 7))
 (segment (start 152.273 76.962) (end 153.797 78.486) (width 0.762) (layer B.Cu) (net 7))
 (segment (start 151.13 76.962) (end 152.273 76.962) (width 0.762) (layer B.Cu) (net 7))
 (segment (start 147.574 109.982) (end 147.574 74.53737) (width 0.762) (layer B.Cu) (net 7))
 (segment (start 144.78 61.722) (end 144.78 64.262) (width 0.762) (layer B.Cu) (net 9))
 (segment (start 145.034 112.014) (end 143.51 112.014) (width 0.762) (layer B.Cu) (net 9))
 (segment (start 146.05 110.998) (end 145.034 112.014) (width 0.762) (layer B.Cu) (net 9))
 (segment (start 144.78 64.262) (end 144.78 65.464081) (width 0.762) (layer B.Cu) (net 9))
 (segment (start 144.78 65.464081) (end 146.05 66.734081) (width 0.762) (layer B.Cu) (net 9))
 (segment (start 146.05 80.63337) (end 146.05 80.01) (width 0.762) (layer B.Cu) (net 9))
 (segment (start 143.51 82.042) (end 144.64137 82.042) (width 0.762) (layer B.Cu) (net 9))
 (segment (start 146.05 66.734081) (end 146.05 80.01) (width 0.762) (layer B.Cu) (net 9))
 (segment (start 144.64137 82.042) (end 146.05 80.63337) (width 0.762) (layer B.Cu) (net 9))
 (segment (start 146.05 110.998) (end 146.05 80.63337) (width 0.762) (layer B.Cu) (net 9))
 (segment (start 143.51 119.634) (end 143.51 117.094) (width 0.762) (layer B.Cu) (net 10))
 (segment (start 138.176 117.094) (end 135.382 114.3) (width 0.762) (layer B.Cu) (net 10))
 (segment (start 143.51 117.094) (end 138.176 117.094) (width 0.762) (layer B.Cu) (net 10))
 (segment (start 135.128 114.046) (end 135.382 114.3) (width 0.762) (layer B.Cu) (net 10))
 (segment (start 135.128 111.252) (end 135.128 114.046) (width 0.762) (layer B.Cu) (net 10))
 (segment (start 162.159001 80.283999) (end 163.957 78.486) (width 0.762) (layer B.Cu) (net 8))
 (segment (start 157.861 104.394) (end 157.861 94.361) (width 0.762) (layer B.Cu) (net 8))
 (segment (start 156.591 105.664) (end 157.861 104.394) (width 0.762) (layer B.Cu) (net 8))
 (segment (start 154.178 105.664) (end 156.591 105.664) (width 0.762) (layer B.Cu) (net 8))
 (segment (start 152.908 106.934) (end 154.178 105.664) (width 0.762) (layer B.Cu) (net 8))
 (segment (start 159.512 92.71) (end 161.671 92.71) (width 0.762) (layer B.Cu) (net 8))
 (segment (start 155.194 122.047) (end 159.111001 118.129999) (width 0.762) (layer B.Cu) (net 8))
 (segment (start 157.353882 109.474) (end 154.051 109.474) (width 0.762) (layer B.Cu) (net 8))
 (segment (start 161.671 92.71) (end 162.159001 92.221999) (width 0.762) (layer B.Cu) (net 8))
 (segment (start 157.861 94.361) (end 159.512 92.71) (width 0.762) (layer B.Cu) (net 8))
 (segment (start 152.908 108.331) (end 152.908 106.934) (width 0.762) (layer B.Cu) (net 8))
 (segment (start 159.111001 111.231119) (end 157.353882 109.474) (width 0.762) (layer B.Cu) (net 8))
 (segment (start 162.159001 92.221999) (end 162.159001 80.283999) (width 0.762) (layer B.Cu) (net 8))
 (segment (start 154.051 109.474) (end 152.908 108.331) (width 0.762) (layer B.Cu) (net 8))
 (segment (start 158.349001 114.554) (end 159.111001 113.792) (width 0.762) (layer B.Cu) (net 8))
 (segment (start 151.13 114.554) (end 158.349001 114.554) (width 0.762) (layer B.Cu) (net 8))
 (segment (start 159.111001 118.129999) (end 159.111001 113.792) (width 0.762) (layer B.Cu) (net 8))
 (segment (start 159.111001 113.792) (end 159.111001 111.231119) (width 0.762) (layer B.Cu) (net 8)))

